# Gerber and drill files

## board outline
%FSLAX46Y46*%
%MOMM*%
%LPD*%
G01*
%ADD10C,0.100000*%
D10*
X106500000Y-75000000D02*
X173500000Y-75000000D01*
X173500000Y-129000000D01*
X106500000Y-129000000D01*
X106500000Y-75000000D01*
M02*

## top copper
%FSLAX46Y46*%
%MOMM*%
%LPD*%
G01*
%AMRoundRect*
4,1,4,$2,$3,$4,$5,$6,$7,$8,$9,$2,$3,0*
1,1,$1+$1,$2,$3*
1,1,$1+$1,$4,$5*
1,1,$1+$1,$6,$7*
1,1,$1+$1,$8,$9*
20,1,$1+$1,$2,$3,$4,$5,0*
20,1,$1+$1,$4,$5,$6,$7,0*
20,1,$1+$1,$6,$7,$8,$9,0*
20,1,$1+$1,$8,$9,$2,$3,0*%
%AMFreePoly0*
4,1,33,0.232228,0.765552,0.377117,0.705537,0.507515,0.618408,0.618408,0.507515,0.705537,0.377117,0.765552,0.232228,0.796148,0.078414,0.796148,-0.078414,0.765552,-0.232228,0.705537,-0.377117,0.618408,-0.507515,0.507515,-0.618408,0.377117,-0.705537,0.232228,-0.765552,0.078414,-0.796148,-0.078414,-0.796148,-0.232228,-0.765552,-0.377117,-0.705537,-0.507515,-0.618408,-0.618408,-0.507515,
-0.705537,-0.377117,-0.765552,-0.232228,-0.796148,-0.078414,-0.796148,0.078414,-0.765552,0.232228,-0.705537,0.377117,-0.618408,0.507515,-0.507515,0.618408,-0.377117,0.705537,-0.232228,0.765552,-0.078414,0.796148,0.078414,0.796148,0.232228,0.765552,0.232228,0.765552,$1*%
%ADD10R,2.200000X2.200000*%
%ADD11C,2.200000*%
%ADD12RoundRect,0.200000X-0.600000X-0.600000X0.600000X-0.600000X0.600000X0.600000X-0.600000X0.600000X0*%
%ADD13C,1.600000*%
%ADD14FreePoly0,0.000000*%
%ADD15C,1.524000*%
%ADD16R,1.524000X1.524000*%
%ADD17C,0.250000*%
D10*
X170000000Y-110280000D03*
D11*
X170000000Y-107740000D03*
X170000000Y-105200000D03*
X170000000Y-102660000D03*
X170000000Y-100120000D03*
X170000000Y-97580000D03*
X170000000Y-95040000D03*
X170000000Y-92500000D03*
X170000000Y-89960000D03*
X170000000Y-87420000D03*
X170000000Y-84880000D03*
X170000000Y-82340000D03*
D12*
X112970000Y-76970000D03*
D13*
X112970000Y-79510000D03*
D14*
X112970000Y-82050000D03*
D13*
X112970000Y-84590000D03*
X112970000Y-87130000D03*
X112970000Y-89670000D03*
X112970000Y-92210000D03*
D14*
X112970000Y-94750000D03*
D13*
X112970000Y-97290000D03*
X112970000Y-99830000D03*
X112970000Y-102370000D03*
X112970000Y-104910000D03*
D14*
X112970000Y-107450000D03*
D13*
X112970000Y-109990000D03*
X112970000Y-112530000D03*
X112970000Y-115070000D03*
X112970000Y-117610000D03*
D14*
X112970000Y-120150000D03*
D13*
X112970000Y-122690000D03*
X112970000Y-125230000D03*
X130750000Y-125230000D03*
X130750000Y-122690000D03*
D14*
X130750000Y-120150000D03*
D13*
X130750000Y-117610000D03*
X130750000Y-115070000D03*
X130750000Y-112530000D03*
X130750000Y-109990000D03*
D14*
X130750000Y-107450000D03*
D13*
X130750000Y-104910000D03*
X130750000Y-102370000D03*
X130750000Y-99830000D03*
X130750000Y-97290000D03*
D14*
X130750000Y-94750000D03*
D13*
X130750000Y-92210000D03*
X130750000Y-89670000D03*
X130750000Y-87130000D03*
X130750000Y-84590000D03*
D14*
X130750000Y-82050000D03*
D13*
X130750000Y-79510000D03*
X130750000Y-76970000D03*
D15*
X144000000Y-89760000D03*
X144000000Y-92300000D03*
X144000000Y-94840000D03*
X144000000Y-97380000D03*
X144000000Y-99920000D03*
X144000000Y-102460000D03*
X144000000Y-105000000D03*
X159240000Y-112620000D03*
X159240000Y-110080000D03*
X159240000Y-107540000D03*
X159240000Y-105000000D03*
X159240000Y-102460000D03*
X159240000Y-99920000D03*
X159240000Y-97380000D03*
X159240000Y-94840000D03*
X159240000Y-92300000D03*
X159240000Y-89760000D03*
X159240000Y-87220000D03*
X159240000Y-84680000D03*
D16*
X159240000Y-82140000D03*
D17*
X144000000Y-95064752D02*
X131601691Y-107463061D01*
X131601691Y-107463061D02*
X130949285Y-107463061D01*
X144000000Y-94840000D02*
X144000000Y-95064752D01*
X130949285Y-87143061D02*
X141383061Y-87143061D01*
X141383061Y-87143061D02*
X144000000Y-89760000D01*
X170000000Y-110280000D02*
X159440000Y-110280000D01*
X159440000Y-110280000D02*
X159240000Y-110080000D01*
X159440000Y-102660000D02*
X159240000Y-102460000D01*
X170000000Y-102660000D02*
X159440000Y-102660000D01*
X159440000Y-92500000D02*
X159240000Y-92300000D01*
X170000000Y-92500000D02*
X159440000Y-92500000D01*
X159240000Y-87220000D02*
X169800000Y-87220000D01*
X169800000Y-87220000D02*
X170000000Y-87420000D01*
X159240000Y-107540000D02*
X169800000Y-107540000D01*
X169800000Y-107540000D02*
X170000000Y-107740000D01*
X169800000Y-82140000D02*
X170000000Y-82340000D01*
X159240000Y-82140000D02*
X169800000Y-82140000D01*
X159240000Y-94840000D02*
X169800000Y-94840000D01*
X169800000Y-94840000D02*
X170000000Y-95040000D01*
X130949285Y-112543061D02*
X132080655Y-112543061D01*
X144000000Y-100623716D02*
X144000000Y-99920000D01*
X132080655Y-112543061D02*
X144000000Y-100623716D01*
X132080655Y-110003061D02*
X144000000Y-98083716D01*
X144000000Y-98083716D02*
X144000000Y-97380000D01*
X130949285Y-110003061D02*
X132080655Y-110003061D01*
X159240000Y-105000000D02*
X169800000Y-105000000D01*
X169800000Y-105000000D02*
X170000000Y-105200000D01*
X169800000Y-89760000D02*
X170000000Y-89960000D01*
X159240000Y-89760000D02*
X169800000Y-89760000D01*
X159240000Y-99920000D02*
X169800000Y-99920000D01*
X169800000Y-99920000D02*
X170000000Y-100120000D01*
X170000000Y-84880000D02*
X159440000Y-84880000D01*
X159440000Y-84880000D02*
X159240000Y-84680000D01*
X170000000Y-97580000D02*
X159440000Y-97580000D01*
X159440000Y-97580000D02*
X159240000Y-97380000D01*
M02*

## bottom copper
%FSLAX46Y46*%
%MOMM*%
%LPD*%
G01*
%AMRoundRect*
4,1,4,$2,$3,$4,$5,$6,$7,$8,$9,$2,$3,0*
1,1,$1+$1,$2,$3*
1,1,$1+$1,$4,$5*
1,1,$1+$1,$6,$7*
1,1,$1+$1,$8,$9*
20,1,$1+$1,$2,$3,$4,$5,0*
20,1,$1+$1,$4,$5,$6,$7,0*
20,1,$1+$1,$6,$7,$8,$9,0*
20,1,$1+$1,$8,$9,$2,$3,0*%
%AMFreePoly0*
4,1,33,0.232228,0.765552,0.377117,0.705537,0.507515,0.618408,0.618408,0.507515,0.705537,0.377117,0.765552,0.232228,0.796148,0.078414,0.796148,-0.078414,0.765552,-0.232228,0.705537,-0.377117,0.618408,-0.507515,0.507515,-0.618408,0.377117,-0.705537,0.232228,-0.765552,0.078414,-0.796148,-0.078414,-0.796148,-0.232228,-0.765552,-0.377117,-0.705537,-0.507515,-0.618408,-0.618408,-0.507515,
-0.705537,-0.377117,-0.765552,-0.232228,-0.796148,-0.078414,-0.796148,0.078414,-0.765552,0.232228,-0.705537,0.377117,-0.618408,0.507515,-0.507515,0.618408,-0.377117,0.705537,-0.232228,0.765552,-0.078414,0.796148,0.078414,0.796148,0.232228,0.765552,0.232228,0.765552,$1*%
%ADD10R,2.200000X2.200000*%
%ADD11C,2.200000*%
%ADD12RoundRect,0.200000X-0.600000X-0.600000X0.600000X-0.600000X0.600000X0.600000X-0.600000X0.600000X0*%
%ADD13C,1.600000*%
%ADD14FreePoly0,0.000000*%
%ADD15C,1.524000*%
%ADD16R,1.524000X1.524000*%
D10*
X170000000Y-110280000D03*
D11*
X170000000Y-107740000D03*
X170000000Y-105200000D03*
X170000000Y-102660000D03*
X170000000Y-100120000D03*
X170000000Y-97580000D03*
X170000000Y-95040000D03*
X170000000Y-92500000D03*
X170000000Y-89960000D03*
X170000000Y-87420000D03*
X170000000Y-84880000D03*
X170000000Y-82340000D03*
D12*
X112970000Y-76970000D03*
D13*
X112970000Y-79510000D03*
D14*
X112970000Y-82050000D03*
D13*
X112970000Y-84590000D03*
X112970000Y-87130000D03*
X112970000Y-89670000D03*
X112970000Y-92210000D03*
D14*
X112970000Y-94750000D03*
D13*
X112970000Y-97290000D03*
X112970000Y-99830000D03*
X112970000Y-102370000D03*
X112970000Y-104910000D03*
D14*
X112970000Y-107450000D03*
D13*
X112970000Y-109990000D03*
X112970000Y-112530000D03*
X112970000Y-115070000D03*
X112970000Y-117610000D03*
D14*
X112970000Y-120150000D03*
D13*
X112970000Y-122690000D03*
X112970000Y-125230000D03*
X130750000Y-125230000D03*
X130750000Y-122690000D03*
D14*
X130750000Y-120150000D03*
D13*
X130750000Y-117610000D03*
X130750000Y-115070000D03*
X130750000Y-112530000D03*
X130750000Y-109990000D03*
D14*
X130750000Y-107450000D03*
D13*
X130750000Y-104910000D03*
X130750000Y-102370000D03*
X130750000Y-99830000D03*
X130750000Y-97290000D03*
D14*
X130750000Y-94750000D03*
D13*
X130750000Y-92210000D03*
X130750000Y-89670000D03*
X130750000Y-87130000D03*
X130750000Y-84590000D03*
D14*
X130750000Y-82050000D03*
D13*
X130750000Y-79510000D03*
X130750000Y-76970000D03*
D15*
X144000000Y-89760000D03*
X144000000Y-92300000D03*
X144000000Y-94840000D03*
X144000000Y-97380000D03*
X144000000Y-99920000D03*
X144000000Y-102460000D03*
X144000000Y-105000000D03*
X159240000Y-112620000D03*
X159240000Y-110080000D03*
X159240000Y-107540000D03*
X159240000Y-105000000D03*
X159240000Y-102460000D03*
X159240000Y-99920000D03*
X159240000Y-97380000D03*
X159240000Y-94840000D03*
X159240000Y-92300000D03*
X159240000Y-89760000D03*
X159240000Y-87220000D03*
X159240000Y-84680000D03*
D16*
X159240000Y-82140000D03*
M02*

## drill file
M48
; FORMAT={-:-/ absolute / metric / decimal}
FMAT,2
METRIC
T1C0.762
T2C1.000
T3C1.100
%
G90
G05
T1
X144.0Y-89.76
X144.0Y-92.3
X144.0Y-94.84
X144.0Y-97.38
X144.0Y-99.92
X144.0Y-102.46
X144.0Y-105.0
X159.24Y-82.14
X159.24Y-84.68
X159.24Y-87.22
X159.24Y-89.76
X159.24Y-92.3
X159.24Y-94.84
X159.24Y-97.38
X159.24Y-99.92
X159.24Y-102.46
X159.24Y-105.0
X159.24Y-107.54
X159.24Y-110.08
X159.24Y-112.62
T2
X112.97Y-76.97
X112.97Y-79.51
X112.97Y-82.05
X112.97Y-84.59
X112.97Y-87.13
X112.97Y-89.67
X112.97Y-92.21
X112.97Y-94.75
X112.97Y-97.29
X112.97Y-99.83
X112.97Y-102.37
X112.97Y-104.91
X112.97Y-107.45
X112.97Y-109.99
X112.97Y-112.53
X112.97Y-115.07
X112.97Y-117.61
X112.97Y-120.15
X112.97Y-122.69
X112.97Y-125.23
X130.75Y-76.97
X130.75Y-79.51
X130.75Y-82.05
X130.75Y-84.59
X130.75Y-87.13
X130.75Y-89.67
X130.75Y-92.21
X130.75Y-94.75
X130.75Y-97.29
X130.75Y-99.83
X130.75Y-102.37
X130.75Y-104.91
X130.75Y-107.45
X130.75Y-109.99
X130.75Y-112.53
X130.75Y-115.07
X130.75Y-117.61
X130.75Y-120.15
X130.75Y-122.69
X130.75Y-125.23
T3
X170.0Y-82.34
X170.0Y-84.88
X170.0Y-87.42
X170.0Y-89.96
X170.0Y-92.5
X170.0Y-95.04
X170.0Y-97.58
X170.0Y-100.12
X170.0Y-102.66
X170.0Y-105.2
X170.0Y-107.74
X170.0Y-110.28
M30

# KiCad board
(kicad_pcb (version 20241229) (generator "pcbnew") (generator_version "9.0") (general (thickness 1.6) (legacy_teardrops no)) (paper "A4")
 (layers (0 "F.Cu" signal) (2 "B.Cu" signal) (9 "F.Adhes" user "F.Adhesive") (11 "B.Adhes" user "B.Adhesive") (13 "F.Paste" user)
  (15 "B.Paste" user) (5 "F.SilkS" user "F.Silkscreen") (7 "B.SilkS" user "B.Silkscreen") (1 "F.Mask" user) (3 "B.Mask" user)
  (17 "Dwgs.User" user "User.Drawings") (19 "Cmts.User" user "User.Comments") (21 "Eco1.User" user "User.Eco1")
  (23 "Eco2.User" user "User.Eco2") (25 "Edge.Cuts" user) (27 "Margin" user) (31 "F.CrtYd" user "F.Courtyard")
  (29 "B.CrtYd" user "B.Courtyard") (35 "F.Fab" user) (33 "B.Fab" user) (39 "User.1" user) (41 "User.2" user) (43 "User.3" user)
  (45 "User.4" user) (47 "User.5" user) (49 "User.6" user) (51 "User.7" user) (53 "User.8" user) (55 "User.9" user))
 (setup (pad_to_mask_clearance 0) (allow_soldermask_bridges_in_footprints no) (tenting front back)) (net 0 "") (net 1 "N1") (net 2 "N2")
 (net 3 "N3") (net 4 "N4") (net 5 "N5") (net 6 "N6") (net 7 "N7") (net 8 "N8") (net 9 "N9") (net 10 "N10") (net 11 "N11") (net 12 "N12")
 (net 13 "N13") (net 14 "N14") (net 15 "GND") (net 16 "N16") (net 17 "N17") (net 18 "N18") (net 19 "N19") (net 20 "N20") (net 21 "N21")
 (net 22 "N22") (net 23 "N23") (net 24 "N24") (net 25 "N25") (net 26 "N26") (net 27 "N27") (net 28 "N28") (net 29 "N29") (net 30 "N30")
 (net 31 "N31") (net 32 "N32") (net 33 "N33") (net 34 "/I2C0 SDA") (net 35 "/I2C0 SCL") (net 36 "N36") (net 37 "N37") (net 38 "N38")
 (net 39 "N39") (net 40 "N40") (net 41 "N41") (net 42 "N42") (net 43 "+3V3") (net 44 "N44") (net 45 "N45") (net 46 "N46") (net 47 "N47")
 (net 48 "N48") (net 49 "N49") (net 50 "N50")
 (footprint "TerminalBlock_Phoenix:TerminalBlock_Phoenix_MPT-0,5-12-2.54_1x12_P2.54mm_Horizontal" (layer "F.Cu") (at 170 110.28 90)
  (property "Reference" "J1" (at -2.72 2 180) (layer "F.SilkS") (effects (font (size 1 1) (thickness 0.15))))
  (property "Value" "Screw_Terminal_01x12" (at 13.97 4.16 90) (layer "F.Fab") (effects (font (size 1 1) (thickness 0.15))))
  (pad "1" thru_hole rect (at 0 0 90) (size 2.2 2.2) (drill 1.1) (layers "*.Cu" "*.Mask") (remove_unused_layers no) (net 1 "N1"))
  (pad "2" thru_hole circle (at 2.54 0 90) (size 2.2 2.2) (drill 1.1) (layers "*.Cu" "*.Mask") (remove_unused_layers no) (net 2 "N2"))
  (pad "3" thru_hole circle (at 5.08 0 90) (size 2.2 2.2) (drill 1.1) (layers "*.Cu" "*.Mask") (remove_unused_layers no) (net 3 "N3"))
  (pad "4" thru_hole circle (at 7.62 0 90) (size 2.2 2.2) (drill 1.1) (layers "*.Cu" "*.Mask") (remove_unused_layers no) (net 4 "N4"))
  (pad "5" thru_hole circle (at 10.16 0 90) (size 2.2 2.2) (drill 1.1) (layers "*.Cu" "*.Mask") (remove_unused_layers no) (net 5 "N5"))
  (pad "6" thru_hole circle (at 12.7 0 90) (size 2.2 2.2) (drill 1.1) (layers "*.Cu" "*.Mask") (remove_unused_layers no) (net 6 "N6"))
  (pad "7" thru_hole circle (at 15.24 0 90) (size 2.2 2.2) (drill 1.1) (layers "*.Cu" "*.Mask") (remove_unused_layers no) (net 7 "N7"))
  (pad "8" thru_hole circle (at 17.78 0 90) (size 2.2 2.2) (drill 1.1) (layers "*.Cu" "*.Mask") (remove_unused_layers no) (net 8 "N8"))
  (pad "9" thru_hole circle (at 20.32 0 90) (size 2.2 2.2) (drill 1.1) (layers "*.Cu" "*.Mask") (remove_unused_layers no) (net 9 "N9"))
  (pad "10" thru_hole circle (at 22.86 0 90) (size 2.2 2.2) (drill 1.1) (layers "*.Cu" "*.Mask") (remove_unused_layers no) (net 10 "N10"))
  (pad "11" thru_hole circle (at 25.4 0 90) (size 2.2 2.2) (drill 1.1) (layers "*.Cu" "*.Mask") (remove_unused_layers no) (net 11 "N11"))
  (pad "12" thru_hole circle (at 27.94 0 90) (size 2.2 2.2) (drill 1.1) (layers "*.Cu" "*.Mask") (remove_unused_layers no) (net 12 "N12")))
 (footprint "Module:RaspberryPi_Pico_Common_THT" (layer "F.Cu") (at 112.97 76.97)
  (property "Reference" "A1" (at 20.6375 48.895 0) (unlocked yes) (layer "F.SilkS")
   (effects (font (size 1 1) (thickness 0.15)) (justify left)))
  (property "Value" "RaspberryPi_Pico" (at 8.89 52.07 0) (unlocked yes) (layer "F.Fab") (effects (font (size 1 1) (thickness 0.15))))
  (pad "1" thru_hole roundrect (at 0 0) (size 1.6 1.6) (drill 1) (layers "*.Cu" "*.Mask") (remove_unused_layers no) (roundrect_rratio 0.125)
   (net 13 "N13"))
  (pad "2" thru_hole circle (at 0 2.54) (size 1.6 1.6) (drill 1) (layers "*.Cu" "*.Mask") (remove_unused_layers no) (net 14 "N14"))
  (pad "3" thru_hole custom (at 0 5.08) (size 1.6 1.6) (drill 1) (layers "*.Cu" "*.Mask") (remove_unused_layers no) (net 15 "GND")
   (options (clearance outline) (anchor circle)) (primitives))
  (pad "4" thru_hole circle (at 0 7.62) (size 1.6 1.6) (drill 1) (layers "*.Cu" "*.Mask") (remove_unused_layers no) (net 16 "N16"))
  (pad "5" thru_hole circle (at 0 10.16) (size 1.6 1.6) (drill 1) (layers "*.Cu" "*.Mask") (remove_unused_layers no) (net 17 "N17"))
  (pad "6" thru_hole circle (at 0 12.7) (size 1.6 1.6) (drill 1) (layers "*.Cu" "*.Mask") (remove_unused_layers no) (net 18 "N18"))
  (pad "7" thru_hole circle (at 0 15.24) (size 1.6 1.6) (drill 1) (layers "*.Cu" "*.Mask") (remove_unused_layers no) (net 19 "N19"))
  (pad "8" thru_hole custom (at 0 17.78) (size 1.6 1.6) (drill 1) (layers "*.Cu" "*.Mask") (remove_unused_layers no) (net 15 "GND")
   (options (clearance outline) (anchor circle)) (primitives))
  (pad "9" thru_hole circle (at 0 20.32) (size 1.6 1.6) (drill 1) (layers "*.Cu" "*.Mask") (remove_unused_layers no) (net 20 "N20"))
  (pad "10" thru_hole circle (at 0 22.86) (size 1.6 1.6) (drill 1) (layers "*.Cu" "*.Mask") (remove_unused_layers no) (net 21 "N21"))
  (pad "11" thru_hole circle (at 0 25.4) (size 1.6 1.6) (drill 1) (layers "*.Cu" "*.Mask") (remove_unused_layers no) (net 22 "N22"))
  (pad "12" thru_hole circle (at 0 27.94) (size 1.6 1.6) (drill 1) (layers "*.Cu" "*.Mask") (remove_unused_layers no) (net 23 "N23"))
  (pad "13" thru_hole custom (at 0 30.48) (size 1.6 1.6) (drill 1) (layers "*.Cu" "*.Mask") (remove_unused_layers no) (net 15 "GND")
   (options (clearance outline) (anchor circle)) (primitives))
  (pad "14" thru_hole circle (at 0 33.02) (size 1.6 1.6) (drill 1) (layers "*.Cu" "*.Mask") (remove_unused_layers no) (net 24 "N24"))
  (pad "15" thru_hole circle (at 0 35.56) (size 1.6 1.6) (drill 1) (layers "*.Cu" "*.Mask") (remove_unused_layers no) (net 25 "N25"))
  (pad "16" thru_hole circle (at 0 38.1) (size 1.6 1.6) (drill 1) (layers "*.Cu" "*.Mask") (remove_unused_layers no) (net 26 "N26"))
  (pad "17" thru_hole circle (at 0 40.64) (size 1.6 1.6) (drill 1) (layers "*.Cu" "*.Mask") (remove_unused_layers no) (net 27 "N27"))
  (pad "18" thru_hole custom (at 0 43.18) (size 1.6 1.6) (drill 1) (layers "*.Cu" "*.Mask") (remove_unused_layers no) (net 15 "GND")
   (options (clearance outline) (anchor circle)) (primitives))
  (pad "19" thru_hole circle (at 0 45.72) (size 1.6 1.6) (drill 1) (layers "*.Cu" "*.Mask") (remove_unused_layers no) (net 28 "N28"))
  (pad "20" thru_hole circle (at 0 48.26) (size 1.6 1.6) (drill 1) (layers "*.Cu" "*.Mask") (remove_unused_layers no) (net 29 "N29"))
  (pad "21" thru_hole circle (at 17.78 48.26) (size 1.6 1.6) (drill 1) (layers "*.Cu" "*.Mask") (remove_unused_layers no) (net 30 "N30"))
  (pad "22" thru_hole circle (at 17.78 45.72) (size 1.6 1.6) (drill 1) (layers "*.Cu" "*.Mask") (remove_unused_layers no) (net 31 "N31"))
  (pad "23" thru_hole custom (at 17.78 43.18) (size 1.6 1.6) (drill 1) (layers "*.Cu" "*.Mask") (remove_unused_layers no) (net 15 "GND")
   (options (clearance outline) (anchor circle)) (primitives))
  (pad "24" thru_hole circle (at 17.78 40.64) (size 1.6 1.6) (drill 1) (layers "*.Cu" "*.Mask") (remove_unused_layers no) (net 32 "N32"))
  (pad "25" thru_hole circle (at 17.78 38.1) (size 1.6 1.6) (drill 1) (layers "*.Cu" "*.Mask") (remove_unused_layers no) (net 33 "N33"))
  (pad "26" thru_hole circle (at 17.78 35.56) (size 1.6 1.6) (drill 1) (layers "*.Cu" "*.Mask") (remove_unused_layers no)
   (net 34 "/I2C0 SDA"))
  (pad "27" thru_hole circle (at 17.78 33.02) (size 1.6 1.6) (drill 1) (layers "*.Cu" "*.Mask") (remove_unused_layers no)
   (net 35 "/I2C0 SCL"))
  (pad "28" thru_hole custom (at 17.78 30.48) (size 1.6 1.6) (drill 1) (layers "*.Cu" "*.Mask") (remove_unused_layers no) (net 15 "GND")
   (options (clearance outline) (anchor circle)) (primitives))
  (pad "29" thru_hole circle (at 17.78 27.94) (size 1.6 1.6) (drill 1) (layers "*.Cu" "*.Mask") (remove_unused_layers no) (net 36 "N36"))
  (pad "30" thru_hole circle (at 17.78 25.4) (size 1.6 1.6) (drill 1) (layers "*.Cu" "*.Mask") (remove_unused_layers no) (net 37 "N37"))
  (pad "31" thru_hole circle (at 17.78 22.86) (size 1.6 1.6) (drill 1) (layers "*.Cu" "*.Mask") (remove_unused_layers no) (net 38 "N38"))
  (pad "32" thru_hole circle (at 17.78 20.32) (size 1.6 1.6) (drill 1) (layers "*.Cu" "*.Mask") (remove_unused_layers no) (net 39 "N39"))
  (pad "33" thru_hole custom (at 17.78 17.78) (size 1.6 1.6) (drill 1) (layers "*.Cu" "*.Mask") (remove_unused_layers no) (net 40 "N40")
   (options (clearance outline) (anchor circle)) (primitives))
  (pad "34" thru_hole circle (at 17.78 15.24) (size 1.6 1.6) (drill 1) (layers "*.Cu" "*.Mask") (remove_unused_layers no) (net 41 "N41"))
  (pad "35" thru_hole circle (at 17.78 12.7) (size 1.6 1.6) (drill 1) (layers "*.Cu" "*.Mask") (remove_unused_layers no) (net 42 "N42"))
  (pad "36" thru_hole circle (at 17.78 10.16) (size 1.6 1.6) (drill 1) (layers "*.Cu" "*.Mask") (remove_unused_layers no) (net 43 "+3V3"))
  (pad "37" thru_hole circle (at 17.78 7.62) (size 1.6 1.6) (drill 1) (layers "*.Cu" "*.Mask") (remove_unused_layers no) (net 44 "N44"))
  (pad "38" thru_hole custom (at 17.78 5.08) (size 1.6 1.6) (drill 1) (layers "*.Cu" "*.Mask") (remove_unused_layers no) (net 15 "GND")
   (options (clearance outline) (anchor circle)) (primitives))
  (pad "39" thru_hole circle (at 17.78 2.54) (size 1.6 1.6) (drill 1) (layers "*.Cu" "*.Mask") (remove_unused_layers no) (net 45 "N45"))
  (pad "40" thru_hole circle (at 17.78 0) (size 1.6 1.6) (drill 1) (layers "*.Cu" "*.Mask") (remove_unused_layers no) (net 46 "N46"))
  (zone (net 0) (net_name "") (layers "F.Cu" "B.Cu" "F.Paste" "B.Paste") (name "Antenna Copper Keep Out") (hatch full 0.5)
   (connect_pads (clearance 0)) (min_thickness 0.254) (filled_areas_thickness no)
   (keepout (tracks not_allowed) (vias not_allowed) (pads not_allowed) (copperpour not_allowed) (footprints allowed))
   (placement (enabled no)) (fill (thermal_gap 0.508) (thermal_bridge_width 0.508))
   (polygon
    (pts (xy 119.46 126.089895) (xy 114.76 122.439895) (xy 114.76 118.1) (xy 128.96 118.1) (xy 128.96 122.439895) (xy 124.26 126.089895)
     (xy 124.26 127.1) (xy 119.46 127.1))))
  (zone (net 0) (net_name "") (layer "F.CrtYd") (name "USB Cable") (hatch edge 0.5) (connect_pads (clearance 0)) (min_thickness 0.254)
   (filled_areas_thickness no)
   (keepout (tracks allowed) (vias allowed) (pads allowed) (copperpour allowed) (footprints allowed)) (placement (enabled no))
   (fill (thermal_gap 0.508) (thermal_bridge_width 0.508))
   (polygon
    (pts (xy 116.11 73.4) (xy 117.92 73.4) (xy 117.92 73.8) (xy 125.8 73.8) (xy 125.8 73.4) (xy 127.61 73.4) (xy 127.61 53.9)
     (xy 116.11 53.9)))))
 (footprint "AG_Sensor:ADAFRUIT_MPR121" (layer "F.Cu") (at 152.89 94.84 -90)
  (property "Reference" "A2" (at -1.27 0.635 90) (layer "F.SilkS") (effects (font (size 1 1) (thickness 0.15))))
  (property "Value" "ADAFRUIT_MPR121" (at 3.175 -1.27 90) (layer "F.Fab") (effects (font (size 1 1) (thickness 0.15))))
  (pad "1" thru_hole circle (at -5.08 8.89 270) (size 1.524 1.524) (drill 0.762) (layers "*.Cu" "*.Mask") (remove_unused_layers no)
   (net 43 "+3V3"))
  (pad "2" thru_hole circle (at -2.54 8.89 270) (size 1.524 1.524) (drill 0.762) (layers "*.Cu" "*.Mask") (remove_unused_layers no)
   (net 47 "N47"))
  (pad "3" thru_hole circle (at 0 8.89 270) (size 1.524 1.524) (drill 0.762) (layers "*.Cu" "*.Mask") (remove_unused_layers no)
   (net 15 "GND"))
  (pad "4" thru_hole circle (at 2.54 8.89 270) (size 1.524 1.524) (drill 0.762) (layers "*.Cu" "*.Mask") (remove_unused_layers no)
   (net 35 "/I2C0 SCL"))
  (pad "5" thru_hole circle (at 5.08 8.89 270) (size 1.524 1.524) (drill 0.762) (layers "*.Cu" "*.Mask") (remove_unused_layers no)
   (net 34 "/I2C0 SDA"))
  (pad "6" thru_hole circle (at 7.62 8.89 270) (size 1.524 1.524) (drill 0.762) (layers "*.Cu" "*.Mask") (remove_unused_layers no)
   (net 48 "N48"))
  (pad "7" thru_hole circle (at 10.16 8.89 270) (size 1.524 1.524) (drill 0.762) (layers "*.Cu" "*.Mask") (remove_unused_layers no)
   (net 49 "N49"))
  (pad "8" thru_hole circle (at 17.78 -6.35 270) (size 1.524 1.524) (drill 0.762) (layers "*.Cu" "*.Mask") (remove_unused_layers no)
   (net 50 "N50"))
  (pad "9" thru_hole circle (at 15.24 -6.35 270) (size 1.524 1.524) (drill 0.762) (layers "*.Cu" "*.Mask") (remove_unused_layers no)
   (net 1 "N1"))
  (pad "10" thru_hole circle (at 12.7 -6.35 270) (size 1.524 1.524) (drill 0.762) (layers "*.Cu" "*.Mask") (remove_unused_layers no)
   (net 2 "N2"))
  (pad "11" thru_hole circle (at 10.16 -6.35) (size 1.524 1.524) (drill 0.762) (layers "*.Cu" "*.Mask") (remove_unused_layers no)
   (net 3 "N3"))
  (pad "12" thru_hole circle (at 7.62 -6.35 270) (size 1.524 1.524) (drill 0.762) (layers "*.Cu" "*.Mask") (remove_unused_layers no)
   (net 4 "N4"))
  (pad "13" thru_hole circle (at 5.08 -6.35 270) (size 1.524 1.524) (drill 0.762) (layers "*.Cu" "*.Mask") (remove_unused_layers no)
   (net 5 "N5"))
  (pad "14" thru_hole circle (at 2.54 -6.35 270) (size 1.524 1.524) (drill 0.762) (layers "*.Cu" "*.Mask") (remove_unused_layers no)
   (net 6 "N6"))
  (pad "15" thru_hole circle (at 0 -6.35 270) (size 1.524 1.524) (drill 0.762) (layers "*.Cu" "*.Mask") (remove_unused_layers no)
   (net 7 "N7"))
  (pad "16" thru_hole circle (at -2.54 -6.35 270) (size 1.524 1.524) (drill 0.762) (layers "*.Cu" "*.Mask") (remove_unused_layers no)
   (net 8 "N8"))
  (pad "17" thru_hole circle (at -5.08 -6.35 270) (size 1.524 1.524) (drill 0.762) (layers "*.Cu" "*.Mask") (remove_unused_layers no)
   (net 9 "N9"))
  (pad "18" thru_hole circle (at -7.62 -6.35 270) (size 1.524 1.524) (drill 0.762) (layers "*.Cu" "*.Mask") (remove_unused_layers no)
   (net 10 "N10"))
  (pad "19" thru_hole circle (at -10.16 -6.35 270) (size 1.524 1.524) (drill 0.762) (layers "*.Cu" "*.Mask") (remove_unused_layers no)
   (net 11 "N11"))
  (pad "20" thru_hole rect (at -12.7 -6.35 270) (size 1.524 1.524) (drill 0.762) (layers "*.Cu" "*.Mask") (remove_unused_layers no)
   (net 12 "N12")))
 (gr_rect (start 106.5 75) (end 173.5 129) (stroke (width 0.1) (type default)) (fill no) (layer "Edge.Cuts"))
 (segment (start 144 95.064752) (end 131.601691 107.463061) (width 0.25) (layer "F.Cu") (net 15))
 (segment (start 131.601691 107.463061) (end 130.949285 107.463061) (width 0.25) (layer "F.Cu") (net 15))
 (segment (start 144 94.84) (end 144 95.064752) (width 0.25) (layer "F.Cu") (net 15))
 (segment (start 130.949285 87.143061) (end 141.383061 87.143061) (width 0.25) (layer "F.Cu") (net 43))
 (segment (start 141.383061 87.143061) (end 144 89.76) (width 0.25) (layer "F.Cu") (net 43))
 (segment (start 170 110.28) (end 159.44 110.28) (width 0.25) (layer "F.Cu") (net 1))
 (segment (start 159.44 110.28) (end 159.24 110.08) (width 0.25) (layer "F.Cu") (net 1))
 (segment (start 159.44 102.66) (end 159.24 102.46) (width 0.25) (layer "F.Cu") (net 4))
 (segment (start 170 102.66) (end 159.44 102.66) (width 0.25) (layer "F.Cu") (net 4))
 (segment (start 159.44 92.5) (end 159.24 92.3) (width 0.25) (layer "F.Cu") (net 8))
 (segment (start 170 92.5) (end 159.44 92.5) (width 0.25) (layer "F.Cu") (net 8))
 (segment (start 159.24 87.22) (end 169.8 87.22) (width 0.25) (layer "F.Cu") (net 10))
 (segment (start 169.8 87.22) (end 170 87.42) (width 0.25) (layer "F.Cu") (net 10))
 (segment (start 159.24 107.54) (end 169.8 107.54) (width 0.25) (layer "F.Cu") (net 2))
 (segment (start 169.8 107.54) (end 170 107.74) (width 0.25) (layer "F.Cu") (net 2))
 (segment (start 169.8 82.14) (end 170 82.34) (width 0.25) (layer "F.Cu") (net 12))
 (segment (start 159.24 82.14) (end 169.8 82.14) (width 0.25) (layer "F.Cu") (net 12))
 (segment (start 159.24 94.84) (end 169.8 94.84) (width 0.25) (layer "F.Cu") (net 7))
 (segment (start 169.8 94.84) (end 170 95.04) (width 0.25) (layer "F.Cu") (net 7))
 (segment (start 130.949285 112.543061) (end 132.080655 112.543061) (width 0.25) (layer "F.Cu") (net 34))
 (segment (start 144 100.623716) (end 144 99.92) (width 0.25) (layer "F.Cu") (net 34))
 (segment (start 132.080655 112.543061) (end 144 100.623716) (width 0.25) (layer "F.Cu") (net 34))
 (segment (start 132.080655 110.003061) (end 144 98.083716) (width 0.25) (layer "F.Cu") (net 35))
 (segment (start 144 98.083716) (end 144 97.38) (width 0.25) (layer "F.Cu") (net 35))
 (segment (start 130.949285 110.003061) (end 132.080655 110.003061) (width 0.25) (layer "F.Cu") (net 35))
 (segment (start 159.24 105) (end 169.8 105) (width 0.25) (layer "F.Cu") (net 3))
 (segment (start 169.8 105) (end 170 105.2) (width 0.25) (layer "F.Cu") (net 3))
 (segment (start 169.8 89.76) (end 170 89.96) (width 0.25) (layer "F.Cu") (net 9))
 (segment (start 159.24 89.76) (end 169.8 89.76) (width 0.25) (layer "F.Cu") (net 9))
 (segment (start 159.24 99.92) (end 169.8 99.92) (width 0.25) (layer "F.Cu") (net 5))
 (segment (start 169.8 99.92) (end 170 100.12) (width 0.25) (layer "F.Cu") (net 5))
 (segment (start 170 84.88) (end 159.44 84.88) (width 0.25) (layer "F.Cu") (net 11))
 (segment (start 159.44 84.88) (end 159.24 84.68) (width 0.25) (layer "F.Cu") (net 11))
 (segment (start 170 97.58) (end 159.44 97.58) (width 0.25) (layer "F.Cu") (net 6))
 (segment (start 159.44 97.58) (end 159.24 97.38) (width 0.25) (layer "F.Cu") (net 6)))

